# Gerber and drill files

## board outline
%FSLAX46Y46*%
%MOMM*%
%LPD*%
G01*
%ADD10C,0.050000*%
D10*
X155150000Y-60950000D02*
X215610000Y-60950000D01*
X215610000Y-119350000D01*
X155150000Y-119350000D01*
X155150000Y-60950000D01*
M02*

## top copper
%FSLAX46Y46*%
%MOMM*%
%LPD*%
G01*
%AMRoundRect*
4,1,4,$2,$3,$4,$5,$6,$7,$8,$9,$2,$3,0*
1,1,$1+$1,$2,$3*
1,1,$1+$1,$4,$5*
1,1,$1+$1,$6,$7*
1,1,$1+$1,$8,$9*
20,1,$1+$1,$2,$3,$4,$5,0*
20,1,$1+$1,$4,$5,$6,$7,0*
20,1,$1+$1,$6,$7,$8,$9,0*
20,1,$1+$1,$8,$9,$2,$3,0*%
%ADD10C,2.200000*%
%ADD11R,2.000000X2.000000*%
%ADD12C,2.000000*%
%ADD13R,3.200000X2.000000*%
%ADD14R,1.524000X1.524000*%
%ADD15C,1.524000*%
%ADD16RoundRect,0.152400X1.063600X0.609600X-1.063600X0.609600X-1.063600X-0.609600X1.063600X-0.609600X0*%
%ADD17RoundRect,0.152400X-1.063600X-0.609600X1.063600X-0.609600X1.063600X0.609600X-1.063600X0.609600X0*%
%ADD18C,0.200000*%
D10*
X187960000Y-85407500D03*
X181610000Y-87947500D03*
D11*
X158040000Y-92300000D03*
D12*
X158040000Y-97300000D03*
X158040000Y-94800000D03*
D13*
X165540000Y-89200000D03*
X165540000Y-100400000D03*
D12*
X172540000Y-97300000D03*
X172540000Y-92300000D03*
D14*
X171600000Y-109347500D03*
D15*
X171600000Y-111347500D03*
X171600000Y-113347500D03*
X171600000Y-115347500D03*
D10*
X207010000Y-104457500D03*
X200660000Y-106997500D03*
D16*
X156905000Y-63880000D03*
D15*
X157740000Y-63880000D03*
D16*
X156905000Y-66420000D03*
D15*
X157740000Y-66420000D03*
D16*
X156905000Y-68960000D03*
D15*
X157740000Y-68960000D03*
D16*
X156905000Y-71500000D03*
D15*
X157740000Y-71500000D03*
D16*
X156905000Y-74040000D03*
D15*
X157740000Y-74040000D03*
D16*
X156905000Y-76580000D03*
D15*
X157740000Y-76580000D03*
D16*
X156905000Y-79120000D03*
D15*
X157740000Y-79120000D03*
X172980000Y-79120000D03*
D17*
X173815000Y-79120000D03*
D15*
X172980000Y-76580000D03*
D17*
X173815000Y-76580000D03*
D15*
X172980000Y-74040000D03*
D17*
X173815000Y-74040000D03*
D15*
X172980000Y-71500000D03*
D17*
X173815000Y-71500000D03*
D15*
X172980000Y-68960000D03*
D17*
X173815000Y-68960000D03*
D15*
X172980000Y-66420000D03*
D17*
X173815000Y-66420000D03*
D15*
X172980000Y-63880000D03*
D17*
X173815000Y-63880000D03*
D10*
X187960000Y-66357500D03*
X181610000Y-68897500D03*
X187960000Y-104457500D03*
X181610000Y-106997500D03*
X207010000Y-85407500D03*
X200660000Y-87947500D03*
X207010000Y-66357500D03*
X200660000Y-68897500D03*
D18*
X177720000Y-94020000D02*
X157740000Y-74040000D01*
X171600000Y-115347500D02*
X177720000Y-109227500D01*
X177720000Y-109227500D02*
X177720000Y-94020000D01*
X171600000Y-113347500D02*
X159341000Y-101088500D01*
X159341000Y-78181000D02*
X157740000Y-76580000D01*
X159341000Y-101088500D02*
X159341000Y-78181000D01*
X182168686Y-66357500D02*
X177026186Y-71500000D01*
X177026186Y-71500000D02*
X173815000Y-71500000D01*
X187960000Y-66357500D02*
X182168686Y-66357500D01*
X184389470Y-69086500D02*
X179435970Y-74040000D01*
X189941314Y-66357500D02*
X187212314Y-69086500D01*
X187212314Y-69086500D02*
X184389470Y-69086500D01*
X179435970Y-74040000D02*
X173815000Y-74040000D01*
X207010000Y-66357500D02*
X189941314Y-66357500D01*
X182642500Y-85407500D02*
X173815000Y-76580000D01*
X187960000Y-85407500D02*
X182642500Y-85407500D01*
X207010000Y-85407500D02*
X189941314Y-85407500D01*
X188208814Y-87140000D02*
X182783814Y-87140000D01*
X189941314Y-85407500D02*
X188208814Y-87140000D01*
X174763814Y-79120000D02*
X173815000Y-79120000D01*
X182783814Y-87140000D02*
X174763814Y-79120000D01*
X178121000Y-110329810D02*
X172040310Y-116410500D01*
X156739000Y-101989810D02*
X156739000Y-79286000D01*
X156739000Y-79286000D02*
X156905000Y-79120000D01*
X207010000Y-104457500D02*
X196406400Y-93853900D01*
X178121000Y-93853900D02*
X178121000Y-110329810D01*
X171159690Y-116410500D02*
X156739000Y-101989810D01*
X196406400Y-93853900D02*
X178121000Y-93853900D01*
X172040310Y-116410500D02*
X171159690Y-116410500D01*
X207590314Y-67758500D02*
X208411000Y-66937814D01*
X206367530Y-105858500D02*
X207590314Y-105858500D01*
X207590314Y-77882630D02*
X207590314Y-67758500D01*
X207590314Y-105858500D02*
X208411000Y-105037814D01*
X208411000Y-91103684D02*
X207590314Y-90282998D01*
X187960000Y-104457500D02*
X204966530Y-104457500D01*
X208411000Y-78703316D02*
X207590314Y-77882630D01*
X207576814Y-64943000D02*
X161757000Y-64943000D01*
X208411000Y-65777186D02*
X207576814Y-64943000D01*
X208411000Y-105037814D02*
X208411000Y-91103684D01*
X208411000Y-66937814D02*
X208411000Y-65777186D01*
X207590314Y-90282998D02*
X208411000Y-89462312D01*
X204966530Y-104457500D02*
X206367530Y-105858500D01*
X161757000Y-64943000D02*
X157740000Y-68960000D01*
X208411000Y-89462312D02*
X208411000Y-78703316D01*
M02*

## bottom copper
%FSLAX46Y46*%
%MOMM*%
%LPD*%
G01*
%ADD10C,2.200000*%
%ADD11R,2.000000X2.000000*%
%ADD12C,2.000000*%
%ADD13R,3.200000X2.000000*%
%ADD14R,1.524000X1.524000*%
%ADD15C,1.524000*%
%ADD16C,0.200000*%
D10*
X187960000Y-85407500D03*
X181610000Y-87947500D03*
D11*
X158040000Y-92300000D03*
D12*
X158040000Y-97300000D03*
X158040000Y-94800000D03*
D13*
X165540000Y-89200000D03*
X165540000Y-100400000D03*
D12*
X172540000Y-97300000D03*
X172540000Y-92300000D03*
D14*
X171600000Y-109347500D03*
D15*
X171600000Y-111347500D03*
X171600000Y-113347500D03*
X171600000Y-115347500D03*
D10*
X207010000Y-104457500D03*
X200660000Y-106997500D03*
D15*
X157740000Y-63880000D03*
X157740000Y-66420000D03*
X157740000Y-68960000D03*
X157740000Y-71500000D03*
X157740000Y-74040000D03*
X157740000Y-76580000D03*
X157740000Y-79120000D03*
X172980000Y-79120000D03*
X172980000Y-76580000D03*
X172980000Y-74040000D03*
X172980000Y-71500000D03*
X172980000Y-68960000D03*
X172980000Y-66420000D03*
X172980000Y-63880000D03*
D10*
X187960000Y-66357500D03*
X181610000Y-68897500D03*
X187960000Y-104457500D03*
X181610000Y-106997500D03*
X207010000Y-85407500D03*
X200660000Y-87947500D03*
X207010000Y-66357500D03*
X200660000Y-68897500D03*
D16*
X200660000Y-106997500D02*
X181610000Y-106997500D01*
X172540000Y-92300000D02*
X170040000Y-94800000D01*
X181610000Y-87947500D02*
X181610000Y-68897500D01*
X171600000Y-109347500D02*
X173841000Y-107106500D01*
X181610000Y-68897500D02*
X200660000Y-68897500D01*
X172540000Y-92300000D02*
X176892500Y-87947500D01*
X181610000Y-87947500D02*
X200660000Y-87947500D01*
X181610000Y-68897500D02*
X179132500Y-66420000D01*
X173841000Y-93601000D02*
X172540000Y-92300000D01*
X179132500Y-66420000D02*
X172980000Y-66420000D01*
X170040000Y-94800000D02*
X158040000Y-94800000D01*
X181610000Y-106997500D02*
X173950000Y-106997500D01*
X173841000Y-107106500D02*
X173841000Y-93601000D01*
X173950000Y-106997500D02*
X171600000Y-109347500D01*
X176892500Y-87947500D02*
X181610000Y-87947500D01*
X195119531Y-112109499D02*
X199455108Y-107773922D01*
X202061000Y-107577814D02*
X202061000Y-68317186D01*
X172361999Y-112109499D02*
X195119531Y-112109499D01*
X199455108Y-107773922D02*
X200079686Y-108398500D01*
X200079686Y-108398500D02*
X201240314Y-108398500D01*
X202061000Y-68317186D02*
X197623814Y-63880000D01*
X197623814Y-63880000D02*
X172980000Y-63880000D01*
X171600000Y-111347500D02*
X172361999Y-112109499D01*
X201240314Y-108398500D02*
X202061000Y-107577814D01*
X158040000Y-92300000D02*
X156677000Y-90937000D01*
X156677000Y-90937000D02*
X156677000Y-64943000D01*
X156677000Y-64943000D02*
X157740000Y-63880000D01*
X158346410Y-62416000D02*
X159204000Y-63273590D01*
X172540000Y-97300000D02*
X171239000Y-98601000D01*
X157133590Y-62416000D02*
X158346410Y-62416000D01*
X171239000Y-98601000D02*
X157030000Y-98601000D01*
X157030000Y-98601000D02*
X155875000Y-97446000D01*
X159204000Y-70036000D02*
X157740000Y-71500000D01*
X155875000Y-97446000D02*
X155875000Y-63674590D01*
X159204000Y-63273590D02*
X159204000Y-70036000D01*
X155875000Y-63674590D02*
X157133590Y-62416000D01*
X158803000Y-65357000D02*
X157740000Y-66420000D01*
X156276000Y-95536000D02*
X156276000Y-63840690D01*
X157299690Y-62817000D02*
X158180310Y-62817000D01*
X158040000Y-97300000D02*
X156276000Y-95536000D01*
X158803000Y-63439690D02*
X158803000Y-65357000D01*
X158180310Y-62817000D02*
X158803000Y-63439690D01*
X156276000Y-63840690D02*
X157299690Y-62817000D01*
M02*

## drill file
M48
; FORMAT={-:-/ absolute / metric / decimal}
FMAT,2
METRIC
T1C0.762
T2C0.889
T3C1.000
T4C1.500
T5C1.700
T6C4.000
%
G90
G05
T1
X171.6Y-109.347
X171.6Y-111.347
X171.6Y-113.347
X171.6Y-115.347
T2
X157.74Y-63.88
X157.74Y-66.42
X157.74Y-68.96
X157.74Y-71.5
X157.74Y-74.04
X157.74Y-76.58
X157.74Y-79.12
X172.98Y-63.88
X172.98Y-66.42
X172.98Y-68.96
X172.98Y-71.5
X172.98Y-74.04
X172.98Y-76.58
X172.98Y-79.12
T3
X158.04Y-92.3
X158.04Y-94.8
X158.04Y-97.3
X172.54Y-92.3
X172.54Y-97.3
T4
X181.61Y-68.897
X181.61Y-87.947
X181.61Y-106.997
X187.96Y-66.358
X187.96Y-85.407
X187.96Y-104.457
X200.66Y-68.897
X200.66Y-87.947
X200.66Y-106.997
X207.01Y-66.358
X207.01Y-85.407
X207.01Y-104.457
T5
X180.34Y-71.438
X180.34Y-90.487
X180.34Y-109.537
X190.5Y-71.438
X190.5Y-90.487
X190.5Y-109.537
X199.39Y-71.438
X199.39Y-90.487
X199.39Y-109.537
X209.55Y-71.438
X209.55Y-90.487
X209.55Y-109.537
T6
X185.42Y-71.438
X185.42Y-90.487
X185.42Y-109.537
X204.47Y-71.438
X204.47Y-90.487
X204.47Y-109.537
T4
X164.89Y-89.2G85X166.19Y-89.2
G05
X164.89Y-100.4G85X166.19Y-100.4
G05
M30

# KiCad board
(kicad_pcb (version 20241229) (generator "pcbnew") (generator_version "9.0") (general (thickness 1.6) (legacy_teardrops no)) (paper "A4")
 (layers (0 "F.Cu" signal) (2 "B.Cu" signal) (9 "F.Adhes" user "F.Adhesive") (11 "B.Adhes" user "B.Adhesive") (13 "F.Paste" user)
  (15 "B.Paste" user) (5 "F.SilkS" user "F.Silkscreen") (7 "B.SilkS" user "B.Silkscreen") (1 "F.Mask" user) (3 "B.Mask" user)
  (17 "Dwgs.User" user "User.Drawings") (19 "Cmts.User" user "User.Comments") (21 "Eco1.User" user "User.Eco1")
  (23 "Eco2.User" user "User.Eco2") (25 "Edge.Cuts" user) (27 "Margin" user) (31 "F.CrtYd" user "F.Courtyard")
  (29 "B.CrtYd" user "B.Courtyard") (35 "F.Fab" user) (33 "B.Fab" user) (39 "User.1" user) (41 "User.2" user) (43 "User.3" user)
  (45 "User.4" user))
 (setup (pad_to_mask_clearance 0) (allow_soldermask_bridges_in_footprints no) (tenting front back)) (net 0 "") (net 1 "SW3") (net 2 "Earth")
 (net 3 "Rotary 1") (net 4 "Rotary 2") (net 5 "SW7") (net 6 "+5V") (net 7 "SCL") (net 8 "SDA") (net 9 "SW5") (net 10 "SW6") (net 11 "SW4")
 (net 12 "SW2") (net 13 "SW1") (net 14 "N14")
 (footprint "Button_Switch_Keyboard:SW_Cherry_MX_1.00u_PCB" (layer "F.Cu") (at 187.96 85.4075)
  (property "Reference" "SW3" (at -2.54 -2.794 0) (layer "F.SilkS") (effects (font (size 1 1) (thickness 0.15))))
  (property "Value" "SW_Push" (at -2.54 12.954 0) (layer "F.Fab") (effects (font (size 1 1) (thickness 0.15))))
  (pad "" np_thru_hole circle (at -7.62 5.08) (size 1.7 1.7) (drill 1.7) (layers "*.Cu" "*.Mask"))
  (pad "" np_thru_hole circle (at -2.54 5.08) (size 4 4) (drill 4) (layers "*.Cu" "*.Mask"))
  (pad "" np_thru_hole circle (at 2.54 5.08) (size 1.7 1.7) (drill 1.7) (layers "*.Cu" "*.Mask"))
  (pad "1" thru_hole circle (at 0 0) (size 2.2 2.2) (drill 1.5) (layers "*.Cu" "*.Mask") (remove_unused_layers no) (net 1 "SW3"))
  (pad "2" thru_hole circle (at -6.35 2.54) (size 2.2 2.2) (drill 1.5) (layers "*.Cu" "*.Mask") (remove_unused_layers no) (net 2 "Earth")))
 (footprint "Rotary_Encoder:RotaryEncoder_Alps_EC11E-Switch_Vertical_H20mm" (layer "F.Cu") (at 158.04 92.3)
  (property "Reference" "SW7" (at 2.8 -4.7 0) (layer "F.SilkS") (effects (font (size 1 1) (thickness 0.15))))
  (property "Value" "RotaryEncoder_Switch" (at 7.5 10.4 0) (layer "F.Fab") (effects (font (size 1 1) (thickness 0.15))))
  (pad "A" thru_hole rect (at 0 0) (size 2 2) (drill 1) (layers "*.Cu" "*.Mask") (remove_unused_layers no) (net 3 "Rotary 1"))
  (pad "B" thru_hole circle (at 0 5) (size 2 2) (drill 1) (layers "*.Cu" "*.Mask") (remove_unused_layers no) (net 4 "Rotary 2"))
  (pad "C" thru_hole circle (at 0 2.5) (size 2 2) (drill 1) (layers "*.Cu" "*.Mask") (remove_unused_layers no) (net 2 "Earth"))
  (pad "MP" thru_hole rect (at 7.5 -3.1) (size 3.2 2) (drill oval 2.8 1.5) (layers "*.Cu" "*.Mask") (remove_unused_layers no))
  (pad "MP" thru_hole rect (at 7.5 8.1) (size 3.2 2) (drill oval 2.8 1.5) (layers "*.Cu" "*.Mask") (remove_unused_layers no))
  (pad "S1" thru_hole circle (at 14.5 5) (size 2 2) (drill 1) (layers "*.Cu" "*.Mask") (remove_unused_layers no) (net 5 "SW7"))
  (pad "S2" thru_hole circle (at 14.5 0) (size 2 2) (drill 1) (layers "*.Cu" "*.Mask") (remove_unused_layers no) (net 2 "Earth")))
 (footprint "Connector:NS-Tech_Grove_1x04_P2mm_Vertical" (layer "F.Cu") (at 171.6 109.3475)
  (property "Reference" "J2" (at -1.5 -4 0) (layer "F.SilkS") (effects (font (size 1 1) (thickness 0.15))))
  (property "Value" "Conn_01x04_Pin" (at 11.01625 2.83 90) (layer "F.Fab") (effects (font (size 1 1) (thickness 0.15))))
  (pad "1" thru_hole rect (at 0 0) (size 1.524 1.524) (drill 0.762) (layers "*.Cu" "*.Mask") (remove_unused_layers no) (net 2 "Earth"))
  (pad "2" thru_hole circle (at 0 2) (size 1.524 1.524) (drill 0.762) (layers "*.Cu" "*.Mask") (remove_unused_layers no) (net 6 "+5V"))
  (pad "3" thru_hole circle (at 0 4) (size 1.524 1.524) (drill 0.762) (layers "*.Cu" "*.Mask") (remove_unused_layers no) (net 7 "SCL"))
  (pad "4" thru_hole circle (at 0 6) (size 1.524 1.524) (drill 0.762) (layers "*.Cu" "*.Mask") (remove_unused_layers no) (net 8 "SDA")))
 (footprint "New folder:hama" (layer "F.Cu") (at 160.55 109.94)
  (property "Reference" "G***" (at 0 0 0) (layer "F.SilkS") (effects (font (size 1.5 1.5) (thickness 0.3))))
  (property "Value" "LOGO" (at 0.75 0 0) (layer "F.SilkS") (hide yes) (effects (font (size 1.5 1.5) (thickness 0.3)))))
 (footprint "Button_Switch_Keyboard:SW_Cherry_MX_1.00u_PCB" (layer "F.Cu") (at 207.01 104.4575)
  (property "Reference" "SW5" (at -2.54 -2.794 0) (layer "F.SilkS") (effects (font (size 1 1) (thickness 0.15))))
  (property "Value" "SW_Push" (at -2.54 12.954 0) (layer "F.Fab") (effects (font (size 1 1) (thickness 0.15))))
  (pad "" np_thru_hole circle (at -7.62 5.08) (size 1.7 1.7) (drill 1.7) (layers "*.Cu" "*.Mask"))
  (pad "" np_thru_hole circle (at -2.54 5.08) (size 4 4) (drill 4) (layers "*.Cu" "*.Mask"))
  (pad "" np_thru_hole circle (at 2.54 5.08) (size 1.7 1.7) (drill 1.7) (layers "*.Cu" "*.Mask"))
  (pad "1" thru_hole circle (at 0 0) (size 2.2 2.2) (drill 1.5) (layers "*.Cu" "*.Mask") (remove_unused_layers no) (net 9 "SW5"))
  (pad "2" thru_hole circle (at -6.35 2.54) (size 2.2 2.2) (drill 1.5) (layers "*.Cu" "*.Mask") (remove_unused_layers no) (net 2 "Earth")))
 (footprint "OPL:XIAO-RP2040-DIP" (layer "F.Cu") (at 165.36 71.5)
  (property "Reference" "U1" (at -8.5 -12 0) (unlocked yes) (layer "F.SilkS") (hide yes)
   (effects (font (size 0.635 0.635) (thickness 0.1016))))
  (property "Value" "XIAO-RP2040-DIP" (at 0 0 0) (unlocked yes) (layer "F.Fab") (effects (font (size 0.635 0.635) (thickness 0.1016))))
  (pad "1" smd roundrect (at -8.455 -7.62 180) (size 2.432 1.524) (layers "F.Cu" "F.Mask") (roundrect_rratio 0.1) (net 3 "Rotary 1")
   (thermal_bridge_angle 45))
  (pad "1" thru_hole circle (at -7.62 -7.62 180) (size 1.524 1.524) (drill 0.889) (layers "*.Cu" "*.Mask") (remove_unused_layers no)
   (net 3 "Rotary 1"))
  (pad "2" smd roundrect (at -8.455 -5.08 180) (size 2.432 1.524) (layers "F.Cu" "F.Mask") (roundrect_rratio 0.1) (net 4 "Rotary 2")
   (thermal_bridge_angle 45))
  (pad "2" thru_hole circle (at -7.62 -5.08 180) (size 1.524 1.524) (drill 0.889) (layers "*.Cu" "*.Mask") (remove_unused_layers no)
   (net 4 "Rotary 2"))
  (pad "3" smd roundrect (at -8.455 -2.54 180) (size 2.432 1.524) (layers "F.Cu" "F.Mask") (roundrect_rratio 0.1) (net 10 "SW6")
   (thermal_bridge_angle 45))
  (pad "3" thru_hole circle (at -7.62 -2.54 180) (size 1.524 1.524) (drill 0.889) (layers "*.Cu" "*.Mask") (remove_unused_layers no)
   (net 10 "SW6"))
  (pad "4" smd roundrect (at -8.455 0 180) (size 2.432 1.524) (layers "F.Cu" "F.Mask") (roundrect_rratio 0.1) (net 5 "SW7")
   (thermal_bridge_angle 45))
  (pad "4" thru_hole circle (at -7.62 0 180) (size 1.524 1.524) (drill 0.889) (layers "*.Cu" "*.Mask") (remove_unused_layers no)
   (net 5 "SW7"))
  (pad "5" smd roundrect (at -8.455 2.54 180) (size 2.432 1.524) (layers "F.Cu" "F.Mask") (roundrect_rratio 0.1) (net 8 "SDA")
   (thermal_bridge_angle 45))
  (pad "5" thru_hole circle (at -7.62 2.54 180) (size 1.524 1.524) (drill 0.889) (layers "*.Cu" "*.Mask") (remove_unused_layers no)
   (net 8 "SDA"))
  (pad "6" smd roundrect (at -8.455 5.08 180) (size 2.432 1.524) (layers "F.Cu" "F.Mask") (roundrect_rratio 0.1) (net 7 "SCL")
   (thermal_bridge_angle 45))
  (pad "6" thru_hole circle (at -7.62 5.08 180) (size 1.524 1.524) (drill 0.889) (layers "*.Cu" "*.Mask") (remove_unused_layers no)
   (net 7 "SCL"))
  (pad "7" smd roundrect (at -8.455 7.62 180) (size 2.432 1.524) (layers "F.Cu" "F.Mask") (roundrect_rratio 0.1) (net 9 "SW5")
   (thermal_bridge_angle 45))
  (pad "7" thru_hole circle (at -7.62 7.62 180) (size 1.524 1.524) (drill 0.889) (layers "*.Cu" "*.Mask") (remove_unused_layers no)
   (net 9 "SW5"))
  (pad "8" thru_hole circle (at 7.62 7.62) (size 1.524 1.524) (drill 0.889) (layers "*.Cu" "*.Mask") (remove_unused_layers no)
   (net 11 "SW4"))
  (pad "8" smd roundrect (at 8.455 7.62) (size 2.432 1.524) (layers "F.Cu" "F.Mask") (roundrect_rratio 0.1) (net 11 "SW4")
   (thermal_bridge_angle 45))
  (pad "9" thru_hole circle (at 7.62 5.08) (size 1.524 1.524) (drill 0.889) (layers "*.Cu" "*.Mask") (remove_unused_layers no) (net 1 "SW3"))
  (pad "9" smd roundrect (at 8.455 5.08) (size 2.432 1.524) (layers "F.Cu" "F.Mask") (roundrect_rratio 0.1) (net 1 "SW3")
   (thermal_bridge_angle 45))
  (pad "10" thru_hole circle (at 7.62 2.54) (size 1.524 1.524) (drill 0.889) (layers "*.Cu" "*.Mask") (remove_unused_layers no)
   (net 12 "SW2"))
  (pad "10" smd roundrect (at 8.455 2.54) (size 2.432 1.524) (layers "F.Cu" "F.Mask") (roundrect_rratio 0.1) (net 12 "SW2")
   (thermal_bridge_angle 45))
  (pad "11" thru_hole circle (at 7.62 0) (size 1.524 1.524) (drill 0.889) (layers "*.Cu" "*.Mask") (remove_unused_layers no) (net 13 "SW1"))
  (pad "11" smd roundrect (at 8.455 0) (size 2.432 1.524) (layers "F.Cu" "F.Mask") (roundrect_rratio 0.1) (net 13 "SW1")
   (thermal_bridge_angle 45))
  (pad "12" thru_hole circle (at 7.62 -2.54) (size 1.524 1.524) (drill 0.889) (layers "*.Cu" "*.Mask") (remove_unused_layers no)
   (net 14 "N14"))
  (pad "12" smd roundrect (at 8.455 -2.54) (size 2.432 1.524) (layers "F.Cu" "F.Mask") (roundrect_rratio 0.1) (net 14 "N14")
   (thermal_bridge_angle 45))
  (pad "13" thru_hole circle (at 7.62 -5.08) (size 1.524 1.524) (drill 0.889) (layers "*.Cu" "*.Mask") (remove_unused_layers no)
   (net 2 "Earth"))
  (pad "13" smd roundrect (at 8.455 -5.08) (size 2.432 1.524) (layers "F.Cu" "F.Mask") (roundrect_rratio 0.1) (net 2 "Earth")
   (thermal_bridge_angle 45))
  (pad "14" thru_hole circle (at 7.62 -7.62) (size 1.524 1.524) (drill 0.889) (layers "*.Cu" "*.Mask") (remove_unused_layers no)
   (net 6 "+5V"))
  (pad "14" smd roundrect (at 8.455 -7.62) (size 2.432 1.524) (layers "F.Cu" "F.Mask") (roundrect_rratio 0.1) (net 6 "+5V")
   (thermal_bridge_angle 45)))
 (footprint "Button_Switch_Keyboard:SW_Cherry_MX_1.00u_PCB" (layer "F.Cu") (at 187.96 66.3575)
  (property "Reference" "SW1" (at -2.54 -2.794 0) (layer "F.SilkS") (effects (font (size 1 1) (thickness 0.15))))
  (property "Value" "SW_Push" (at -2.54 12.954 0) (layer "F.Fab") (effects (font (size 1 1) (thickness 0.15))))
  (pad "" np_thru_hole circle (at -7.62 5.08) (size 1.7 1.7) (drill 1.7) (layers "*.Cu" "*.Mask"))
  (pad "" np_thru_hole circle (at -2.54 5.08) (size 4 4) (drill 4) (layers "*.Cu" "*.Mask"))
  (pad "" np_thru_hole circle (at 2.54 5.08) (size 1.7 1.7) (drill 1.7) (layers "*.Cu" "*.Mask"))
  (pad "1" thru_hole circle (at 0 0) (size 2.2 2.2) (drill 1.5) (layers "*.Cu" "*.Mask") (remove_unused_layers no) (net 13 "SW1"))
  (pad "2" thru_hole circle (at -6.35 2.54) (size 2.2 2.2) (drill 1.5) (layers "*.Cu" "*.Mask") (remove_unused_layers no) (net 2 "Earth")))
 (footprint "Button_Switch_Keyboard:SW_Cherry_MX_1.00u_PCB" (layer "F.Cu") (at 187.96 104.4575)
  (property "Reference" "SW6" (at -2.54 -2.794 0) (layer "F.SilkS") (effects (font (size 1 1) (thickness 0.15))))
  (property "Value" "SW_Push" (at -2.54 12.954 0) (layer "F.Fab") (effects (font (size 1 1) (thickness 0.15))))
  (pad "" np_thru_hole circle (at -7.62 5.08) (size 1.7 1.7) (drill 1.7) (layers "*.Cu" "*.Mask"))
  (pad "" np_thru_hole circle (at -2.54 5.08) (size 4 4) (drill 4) (layers "*.Cu" "*.Mask"))
  (pad "" np_thru_hole circle (at 2.54 5.08) (size 1.7 1.7) (drill 1.7) (layers "*.Cu" "*.Mask"))
  (pad "1" thru_hole circle (at 0 0) (size 2.2 2.2) (drill 1.5) (layers "*.Cu" "*.Mask") (remove_unused_layers no) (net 10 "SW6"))
  (pad "2" thru_hole circle (at -6.35 2.54) (size 2.2 2.2) (drill 1.5) (layers "*.Cu" "*.Mask") (remove_unused_layers no) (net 2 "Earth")))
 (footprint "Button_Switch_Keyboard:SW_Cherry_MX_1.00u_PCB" (layer "F.Cu") (at 207.01 85.4075)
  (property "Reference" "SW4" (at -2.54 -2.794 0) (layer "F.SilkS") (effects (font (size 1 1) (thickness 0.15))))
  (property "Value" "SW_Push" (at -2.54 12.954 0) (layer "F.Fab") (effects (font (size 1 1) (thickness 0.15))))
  (pad "" np_thru_hole circle (at -7.62 5.08) (size 1.7 1.7) (drill 1.7) (layers "*.Cu" "*.Mask"))
  (pad "" np_thru_hole circle (at -2.54 5.08) (size 4 4) (drill 4) (layers "*.Cu" "*.Mask"))
  (pad "" np_thru_hole circle (at 2.54 5.08) (size 1.7 1.7) (drill 1.7) (layers "*.Cu" "*.Mask"))
  (pad "1" thru_hole circle (at 0 0) (size 2.2 2.2) (drill 1.5) (layers "*.Cu" "*.Mask") (remove_unused_layers no) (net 11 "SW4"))
  (pad "2" thru_hole circle (at -6.35 2.54) (size 2.2 2.2) (drill 1.5) (layers "*.Cu" "*.Mask") (remove_unused_layers no) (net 2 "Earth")))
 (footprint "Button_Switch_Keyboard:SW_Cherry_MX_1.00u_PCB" (layer "F.Cu") (at 207.01 66.3575)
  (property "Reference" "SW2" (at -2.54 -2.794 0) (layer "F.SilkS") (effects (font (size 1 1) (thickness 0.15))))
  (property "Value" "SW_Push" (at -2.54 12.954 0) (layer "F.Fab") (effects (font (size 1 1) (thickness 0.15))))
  (pad "" np_thru_hole circle (at -7.62 5.08) (size 1.7 1.7) (drill 1.7) (layers "*.Cu" "*.Mask"))
  (pad "" np_thru_hole circle (at -2.54 5.08) (size 4 4) (drill 4) (layers "*.Cu" "*.Mask"))
  (pad "" np_thru_hole circle (at 2.54 5.08) (size 1.7 1.7) (drill 1.7) (layers "*.Cu" "*.Mask"))
  (pad "1" thru_hole circle (at 0 0) (size 2.2 2.2) (drill 1.5) (layers "*.Cu" "*.Mask") (remove_unused_layers no) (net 12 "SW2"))
  (pad "2" thru_hole circle (at -6.35 2.54) (size 2.2 2.2) (drill 1.5) (layers "*.Cu" "*.Mask") (remove_unused_layers no) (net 2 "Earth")))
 (gr_rect (start 155.15 60.95) (end 215.61 119.35) (stroke (width 0.05) (type default)) (fill no) (layer "Edge.Cuts"))
 (segment (start 200.66 106.9975) (end 181.61 106.9975) (width 0.2) (layer "B.Cu") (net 2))
 (segment (start 172.54 92.3) (end 170.04 94.8) (width 0.2) (layer "B.Cu") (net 2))
 (segment (start 181.61 87.9475) (end 181.61 68.8975) (width 0.2) (layer "B.Cu") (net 2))
 (segment (start 171.6 109.3475) (end 173.841 107.1065) (width 0.2) (layer "B.Cu") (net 2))
 (segment (start 181.61 68.8975) (end 200.66 68.8975) (width 0.2) (layer "B.Cu") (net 2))
 (segment (start 172.54 92.3) (end 176.8925 87.9475) (width 0.2) (layer "B.Cu") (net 2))
 (segment (start 181.61 87.9475) (end 200.66 87.9475) (width 0.2) (layer "B.Cu") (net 2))
 (segment (start 181.61 68.8975) (end 179.1325 66.42) (width 0.2) (layer "B.Cu") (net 2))
 (segment (start 173.841 93.601) (end 172.54 92.3) (width 0.2) (layer "B.Cu") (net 2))
 (segment (start 179.1325 66.42) (end 172.98 66.42) (width 0.2) (layer "B.Cu") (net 2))
 (segment (start 170.04 94.8) (end 158.04 94.8) (width 0.2) (layer "B.Cu") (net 2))
 (segment (start 181.61 106.9975) (end 173.95 106.9975) (width 0.2) (layer "B.Cu") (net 2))
 (segment (start 173.841 107.1065) (end 173.841 93.601) (width 0.2) (layer "B.Cu") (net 2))
 (segment (start 173.95 106.9975) (end 171.6 109.3475) (width 0.2) (layer "B.Cu") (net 2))
 (segment (start 176.8925 87.9475) (end 181.61 87.9475) (width 0.2) (layer "B.Cu") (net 2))
 (segment (start 177.72 94.02) (end 157.74 74.04) (width 0.2) (layer "F.Cu") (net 8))
 (segment (start 171.6 115.3475) (end 177.72 109.2275) (width 0.2) (layer "F.Cu") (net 8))
 (segment (start 177.72 109.2275) (end 177.72 94.02) (width 0.2) (layer "F.Cu") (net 8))
 (segment (start 195.119531 112.109499) (end 199.455108 107.773922) (width 0.2) (layer "B.Cu") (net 6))
 (segment (start 202.061 107.577814) (end 202.061 68.317186) (width 0.2) (layer "B.Cu") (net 6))
 (segment (start 172.361999 112.109499) (end 195.119531 112.109499) (width 0.2) (layer "B.Cu") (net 6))
 (segment (start 199.455108 107.773922) (end 200.079686 108.3985) (width 0.2) (layer "B.Cu") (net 6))
 (segment (start 200.079686 108.3985) (end 201.240314 108.3985) (width 0.2) (layer "B.Cu") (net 6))
 (segment (start 202.061 68.317186) (end 197.623814 63.88) (width 0.2) (layer "B.Cu") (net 6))
 (segment (start 197.623814 63.88) (end 172.98 63.88) (width 0.2) (layer "B.Cu") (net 6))
 (segment (start 171.6 111.3475) (end 172.361999 112.109499) (width 0.2) (layer "B.Cu") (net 6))
 (segment (start 201.240314 108.3985) (end 202.061 107.577814) (width 0.2) (layer "B.Cu") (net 6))
 (segment (start 171.6 113.3475) (end 159.341 101.0885) (width 0.2) (layer "F.Cu") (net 7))
 (segment (start 159.341 78.181) (end 157.74 76.58) (width 0.2) (layer "F.Cu") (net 7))
 (segment (start 159.341 101.0885) (end 159.341 78.181) (width 0.2) (layer "F.Cu") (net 7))
 (segment (start 182.168686 66.3575) (end 177.026186 71.5) (width 0.2) (layer "F.Cu") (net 13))
 (segment (start 177.026186 71.5) (end 173.815 71.5) (width 0.2) (layer "F.Cu") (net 13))
 (segment (start 187.96 66.3575) (end 182.168686 66.3575) (width 0.2) (layer "F.Cu") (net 13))
 (segment (start 184.38947 69.0865) (end 179.43597 74.04) (width 0.2) (layer "F.Cu") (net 12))
 (segment (start 189.941314 66.3575) (end 187.212314 69.0865) (width 0.2) (layer "F.Cu") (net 12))
 (segment (start 187.212314 69.0865) (end 184.38947 69.0865) (width 0.2) (layer "F.Cu") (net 12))
 (segment (start 179.43597 74.04) (end 173.815 74.04) (width 0.2) (layer "F.Cu") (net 12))
 (segment (start 207.01 66.3575) (end 189.941314 66.3575) (width 0.2) (layer "F.Cu") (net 12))
 (segment (start 182.6425 85.4075) (end 173.815 76.58) (width 0.2) (layer "F.Cu") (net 1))
 (segment (start 187.96 85.4075) (end 182.6425 85.4075) (width 0.2) (layer "F.Cu") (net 1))
 (segment (start 207.01 85.4075) (end 189.941314 85.4075) (width 0.2) (layer "F.Cu") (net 11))
 (segment (start 188.208814 87.14) (end 182.783814 87.14) (width 0.2) (layer "F.Cu") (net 11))
 (segment (start 189.941314 85.4075) (end 188.208814 87.14) (width 0.2) (layer "F.Cu") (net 11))
 (segment (start 174.763814 79.12) (end 173.815 79.12) (width 0.2) (layer "F.Cu") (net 11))
 (segment (start 182.783814 87.14) (end 174.763814 79.12) (width 0.2) (layer "F.Cu") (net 11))
 (segment (start 178.121 110.32981) (end 172.04031 116.4105) (width 0.2) (layer "F.Cu") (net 9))
 (segment (start 156.739 101.98981) (end 156.739 79.286) (width 0.2) (layer "F.Cu") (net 9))
 (segment (start 156.739 79.286) (end 156.905 79.12) (width 0.2) (layer "F.Cu") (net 9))
 (segment (start 207.01 104.4575) (end 196.4064 93.8539) (width 0.2) (layer "F.Cu") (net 9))
 (segment (start 178.121 93.8539) (end 178.121 110.32981) (width 0.2) (layer "F.Cu") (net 9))
 (segment (start 171.15969 116.4105) (end 156.739 101.98981) (width 0.2) (layer "F.Cu") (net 9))
 (segment (start 196.4064 93.8539) (end 178.121 93.8539) (width 0.2) (layer "F.Cu") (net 9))
 (segment (start 172.04031 116.4105) (end 171.15969 116.4105) (width 0.2) (layer "F.Cu") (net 9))
 (segment (start 207.590314 67.7585) (end 208.411 66.937814) (width 0.2) (layer "F.Cu") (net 10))
 (segment (start 206.36753 105.8585) (end 207.590314 105.8585) (width 0.2) (layer "F.Cu") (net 10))
 (segment (start 207.590314 77.88263) (end 207.590314 67.7585) (width 0.2) (layer "F.Cu") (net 10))
 (segment (start 207.590314 105.8585) (end 208.411 105.037814) (width 0.2) (layer "F.Cu") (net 10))
 (segment (start 208.411 91.103684) (end 207.590314 90.282998) (width 0.2) (layer "F.Cu") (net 10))
 (segment (start 187.96 104.4575) (end 204.96653 104.4575) (width 0.2) (layer "F.Cu") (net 10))
 (segment (start 208.411 78.703316) (end 207.590314 77.88263) (width 0.2) (layer "F.Cu") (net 10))
 (segment (start 207.576814 64.943) (end 161.757 64.943) (width 0.2) (layer "F.Cu") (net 10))
 (segment (start 208.411 65.777186) (end 207.576814 64.943) (width 0.2) (layer "F.Cu") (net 10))
 (segment (start 208.411 105.037814) (end 208.411 91.103684) (width 0.2) (layer "F.Cu") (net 10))
 (segment (start 208.411 66.937814) (end 208.411 65.777186) (width 0.2) (layer "F.Cu") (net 10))
 (segment (start 207.590314 90.282998) (end 208.411 89.462312) (width 0.2) (layer "F.Cu") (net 10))
 (segment (start 204.96653 104.4575) (end 206.36753 105.8585) (width 0.2) (layer "F.Cu") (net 10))
 (segment (start 161.757 64.943) (end 157.74 68.96) (width 0.2) (layer "F.Cu") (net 10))
 (segment (start 208.411 89.462312) (end 208.411 78.703316) (width 0.2) (layer "F.Cu") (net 10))
 (segment (start 158.04 92.3) (end 156.677 90.937) (width 0.2) (layer "B.Cu") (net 3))
 (segment (start 156.677 90.937) (end 156.677 64.943) (width 0.2) (layer "B.Cu") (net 3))
 (segment (start 156.677 64.943) (end 157.74 63.88) (width 0.2) (layer "B.Cu") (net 3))
 (segment (start 158.34641 62.416) (end 159.204 63.27359) (width 0.2) (layer "B.Cu") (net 5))
 (segment (start 172.54 97.3) (end 171.239 98.601) (width 0.2) (layer "B.Cu") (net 5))
 (segment (start 157.13359 62.416) (end 158.34641 62.416) (width 0.2) (layer "B.Cu") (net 5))
 (segment (start 171.239 98.601) (end 157.03 98.601) (width 0.2) (layer "B.Cu") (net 5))
 (segment (start 157.03 98.601) (end 155.875 97.446) (width 0.2) (layer "B.Cu") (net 5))
 (segment (start 159.204 70.036) (end 157.74 71.5) (width 0.2) (layer "B.Cu") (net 5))
 (segment (start 155.875 97.446) (end 155.875 63.67459) (width 0.2) (layer "B.Cu") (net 5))
 (segment (start 159.204 63.27359) (end 159.204 70.036) (width 0.2) (layer "B.Cu") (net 5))
 (segment (start 155.875 63.67459) (end 157.13359 62.416) (width 0.2) (layer "B.Cu") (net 5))
 (segment (start 158.803 65.357) (end 157.74 66.42) (width 0.2) (layer "B.Cu") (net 4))
 (segment (start 156.276 95.536) (end 156.276 63.84069) (width 0.2) (layer "B.Cu") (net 4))
 (segment (start 157.29969 62.817) (end 158.18031 62.817) (width 0.2) (layer "B.Cu") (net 4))
 (segment (start 158.04 97.3) (end 156.276 95.536) (width 0.2) (layer "B.Cu") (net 4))
 (segment (start 158.803 63.43969) (end 158.803 65.357) (width 0.2) (layer "B.Cu") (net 4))
 (segment (start 158.18031 62.817) (end 158.803 63.43969) (width 0.2) (layer "B.Cu") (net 4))
 (segment (start 156.276 63.84069) (end 157.29969 62.817) (width 0.2) (layer "B.Cu") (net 4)))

